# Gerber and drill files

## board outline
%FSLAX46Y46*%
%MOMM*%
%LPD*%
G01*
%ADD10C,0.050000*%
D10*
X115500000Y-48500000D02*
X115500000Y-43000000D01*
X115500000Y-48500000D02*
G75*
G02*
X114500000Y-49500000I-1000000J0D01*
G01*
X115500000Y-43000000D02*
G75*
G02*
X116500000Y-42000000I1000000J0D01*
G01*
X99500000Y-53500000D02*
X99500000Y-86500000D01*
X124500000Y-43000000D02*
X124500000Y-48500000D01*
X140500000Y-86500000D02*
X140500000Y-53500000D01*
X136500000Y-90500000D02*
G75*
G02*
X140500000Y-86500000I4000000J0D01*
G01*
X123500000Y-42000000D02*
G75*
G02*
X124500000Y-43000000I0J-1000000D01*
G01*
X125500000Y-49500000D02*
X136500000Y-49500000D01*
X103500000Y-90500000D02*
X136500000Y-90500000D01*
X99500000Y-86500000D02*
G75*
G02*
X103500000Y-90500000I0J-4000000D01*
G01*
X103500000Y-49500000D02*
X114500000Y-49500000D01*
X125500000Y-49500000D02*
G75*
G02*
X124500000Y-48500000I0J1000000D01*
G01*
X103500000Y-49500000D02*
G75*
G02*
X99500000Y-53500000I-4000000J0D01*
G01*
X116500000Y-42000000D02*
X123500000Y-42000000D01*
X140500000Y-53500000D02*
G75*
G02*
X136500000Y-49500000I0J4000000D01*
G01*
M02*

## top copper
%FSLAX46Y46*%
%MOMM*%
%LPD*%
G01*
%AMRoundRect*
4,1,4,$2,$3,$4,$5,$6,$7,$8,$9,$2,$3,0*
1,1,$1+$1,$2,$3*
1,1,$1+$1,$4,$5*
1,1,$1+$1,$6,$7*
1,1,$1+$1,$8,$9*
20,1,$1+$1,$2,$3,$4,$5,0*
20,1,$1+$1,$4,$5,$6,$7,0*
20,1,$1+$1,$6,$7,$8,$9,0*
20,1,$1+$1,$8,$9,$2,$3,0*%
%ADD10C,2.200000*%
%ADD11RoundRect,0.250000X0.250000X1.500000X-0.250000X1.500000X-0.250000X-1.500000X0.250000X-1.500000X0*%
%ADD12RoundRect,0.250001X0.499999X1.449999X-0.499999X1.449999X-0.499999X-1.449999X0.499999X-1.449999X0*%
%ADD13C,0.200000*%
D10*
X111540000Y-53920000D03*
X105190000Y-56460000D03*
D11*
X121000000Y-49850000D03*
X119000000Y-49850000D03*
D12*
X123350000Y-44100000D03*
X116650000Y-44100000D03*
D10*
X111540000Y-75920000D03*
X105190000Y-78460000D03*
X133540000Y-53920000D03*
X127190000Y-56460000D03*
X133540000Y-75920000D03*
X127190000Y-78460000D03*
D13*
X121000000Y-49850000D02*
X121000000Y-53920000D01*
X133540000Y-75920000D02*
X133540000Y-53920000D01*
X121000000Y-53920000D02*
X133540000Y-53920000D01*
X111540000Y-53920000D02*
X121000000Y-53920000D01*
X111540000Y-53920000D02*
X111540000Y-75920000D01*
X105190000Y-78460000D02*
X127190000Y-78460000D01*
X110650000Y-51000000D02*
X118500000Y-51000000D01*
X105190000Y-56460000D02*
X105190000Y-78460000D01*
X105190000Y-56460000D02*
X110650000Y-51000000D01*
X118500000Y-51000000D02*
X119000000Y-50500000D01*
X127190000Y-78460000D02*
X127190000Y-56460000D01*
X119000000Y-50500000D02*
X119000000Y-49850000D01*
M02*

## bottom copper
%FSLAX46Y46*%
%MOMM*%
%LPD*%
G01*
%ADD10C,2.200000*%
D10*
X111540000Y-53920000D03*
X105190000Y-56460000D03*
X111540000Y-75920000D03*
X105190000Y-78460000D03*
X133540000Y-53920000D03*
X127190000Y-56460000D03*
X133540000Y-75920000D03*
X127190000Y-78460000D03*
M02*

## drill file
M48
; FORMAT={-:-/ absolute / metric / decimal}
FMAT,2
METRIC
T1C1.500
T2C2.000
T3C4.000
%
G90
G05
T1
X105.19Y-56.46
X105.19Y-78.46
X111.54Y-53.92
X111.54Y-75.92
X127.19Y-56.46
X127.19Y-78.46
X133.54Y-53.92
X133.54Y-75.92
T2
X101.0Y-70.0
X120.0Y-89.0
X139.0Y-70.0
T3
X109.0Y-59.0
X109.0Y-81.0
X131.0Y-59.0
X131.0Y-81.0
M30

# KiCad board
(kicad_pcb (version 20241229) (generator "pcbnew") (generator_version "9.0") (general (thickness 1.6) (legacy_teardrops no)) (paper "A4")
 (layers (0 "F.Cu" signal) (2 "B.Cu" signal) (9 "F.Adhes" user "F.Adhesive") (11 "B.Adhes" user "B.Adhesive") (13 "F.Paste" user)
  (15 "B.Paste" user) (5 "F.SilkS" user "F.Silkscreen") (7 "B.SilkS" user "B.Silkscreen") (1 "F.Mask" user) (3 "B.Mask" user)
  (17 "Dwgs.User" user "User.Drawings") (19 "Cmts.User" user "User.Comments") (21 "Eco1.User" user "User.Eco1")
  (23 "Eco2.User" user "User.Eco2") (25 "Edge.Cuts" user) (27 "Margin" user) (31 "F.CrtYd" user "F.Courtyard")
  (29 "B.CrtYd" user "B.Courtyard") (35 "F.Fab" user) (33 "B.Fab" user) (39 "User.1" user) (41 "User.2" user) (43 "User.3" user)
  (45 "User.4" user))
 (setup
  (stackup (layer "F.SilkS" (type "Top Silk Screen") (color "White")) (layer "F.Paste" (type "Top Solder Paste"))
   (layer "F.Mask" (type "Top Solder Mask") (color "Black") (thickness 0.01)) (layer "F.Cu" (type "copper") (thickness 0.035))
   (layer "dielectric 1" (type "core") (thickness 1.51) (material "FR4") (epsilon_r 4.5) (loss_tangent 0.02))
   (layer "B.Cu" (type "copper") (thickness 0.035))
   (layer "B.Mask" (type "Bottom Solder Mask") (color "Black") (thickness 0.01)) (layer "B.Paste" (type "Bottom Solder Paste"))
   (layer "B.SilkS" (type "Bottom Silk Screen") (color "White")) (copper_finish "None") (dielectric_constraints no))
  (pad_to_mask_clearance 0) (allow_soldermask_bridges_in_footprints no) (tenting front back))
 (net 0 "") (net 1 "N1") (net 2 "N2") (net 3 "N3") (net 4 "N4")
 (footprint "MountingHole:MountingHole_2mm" (layer "F.Cu") (at 139 70)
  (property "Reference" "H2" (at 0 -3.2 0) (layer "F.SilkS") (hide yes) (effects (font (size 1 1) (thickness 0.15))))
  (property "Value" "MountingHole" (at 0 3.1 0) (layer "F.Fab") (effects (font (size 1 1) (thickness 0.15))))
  (pad "" np_thru_hole circle (at 0 0) (size 2 2) (drill 2) (layers "*.Cu" "*.Mask")))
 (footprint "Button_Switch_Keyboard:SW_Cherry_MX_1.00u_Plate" (layer "F.Cu") (at 111.54 53.92)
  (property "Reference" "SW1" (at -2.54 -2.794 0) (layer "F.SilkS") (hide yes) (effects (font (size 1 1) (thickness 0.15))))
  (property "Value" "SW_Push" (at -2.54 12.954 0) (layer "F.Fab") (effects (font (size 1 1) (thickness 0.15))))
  (pad "" np_thru_hole circle (at -2.54 5.08) (size 4 4) (drill 4) (layers "*.Cu" "*.Mask"))
  (pad "1" thru_hole circle (at 0 0) (size 2.2 2.2) (drill 1.5) (layers "*.Cu" "*.Mask") (remove_unused_layers no) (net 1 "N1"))
  (pad "2" thru_hole circle (at -6.35 2.54) (size 2.2 2.2) (drill 1.5) (layers "*.Cu" "*.Mask") (remove_unused_layers no) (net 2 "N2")))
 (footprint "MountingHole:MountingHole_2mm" (layer "F.Cu") (at 120 89)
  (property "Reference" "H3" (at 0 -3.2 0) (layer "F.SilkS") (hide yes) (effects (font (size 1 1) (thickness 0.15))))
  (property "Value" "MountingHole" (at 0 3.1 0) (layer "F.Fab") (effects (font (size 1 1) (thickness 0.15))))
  (pad "" np_thru_hole circle (at 0 0) (size 2 2) (drill 2) (layers "*.Cu" "*.Mask")))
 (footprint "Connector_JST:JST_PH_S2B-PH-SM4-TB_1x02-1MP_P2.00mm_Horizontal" (layer "F.Cu") (at 120 47 180)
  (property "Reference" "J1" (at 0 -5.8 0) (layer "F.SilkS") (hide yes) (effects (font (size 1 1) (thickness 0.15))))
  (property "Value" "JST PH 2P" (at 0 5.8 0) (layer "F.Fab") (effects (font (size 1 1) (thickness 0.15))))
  (pad "1" smd roundrect (at -1 -2.85 180) (size 1 3.5) (layers "F.Cu" "F.Mask" "F.Paste") (roundrect_rratio 0.25) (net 1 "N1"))
  (pad "2" smd roundrect (at 1 -2.85 180) (size 1 3.5) (layers "F.Cu" "F.Mask" "F.Paste") (roundrect_rratio 0.25) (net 2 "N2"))
  (pad "MP" smd roundrect (at -3.35 2.9 180) (size 1.5 3.4) (layers "F.Cu" "F.Mask" "F.Paste") (roundrect_rratio 0.166667) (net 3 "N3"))
  (pad "MP" smd roundrect (at 3.35 2.9 180) (size 1.5 3.4) (layers "F.Cu" "F.Mask" "F.Paste") (roundrect_rratio 0.166667) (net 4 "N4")))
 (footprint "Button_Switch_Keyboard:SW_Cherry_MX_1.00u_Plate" (layer "F.Cu") (at 111.54 75.92)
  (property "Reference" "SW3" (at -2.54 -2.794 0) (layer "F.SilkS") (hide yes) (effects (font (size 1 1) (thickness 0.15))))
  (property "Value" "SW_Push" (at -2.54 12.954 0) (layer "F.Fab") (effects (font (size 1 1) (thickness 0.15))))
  (pad "" np_thru_hole circle (at -2.54 5.08) (size 4 4) (drill 4) (layers "*.Cu" "*.Mask"))
  (pad "1" thru_hole circle (at 0 0) (size 2.2 2.2) (drill 1.5) (layers "*.Cu" "*.Mask") (remove_unused_layers no) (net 1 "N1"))
  (pad "2" thru_hole circle (at -6.35 2.54) (size 2.2 2.2) (drill 1.5) (layers "*.Cu" "*.Mask") (remove_unused_layers no) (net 2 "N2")))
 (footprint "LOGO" (layer "F.Cu") (at 126.5 70.1)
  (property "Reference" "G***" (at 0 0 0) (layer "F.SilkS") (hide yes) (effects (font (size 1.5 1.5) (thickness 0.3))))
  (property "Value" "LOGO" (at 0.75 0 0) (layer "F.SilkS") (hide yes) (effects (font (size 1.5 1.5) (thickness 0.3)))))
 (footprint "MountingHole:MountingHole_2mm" (layer "F.Cu") (at 101 70)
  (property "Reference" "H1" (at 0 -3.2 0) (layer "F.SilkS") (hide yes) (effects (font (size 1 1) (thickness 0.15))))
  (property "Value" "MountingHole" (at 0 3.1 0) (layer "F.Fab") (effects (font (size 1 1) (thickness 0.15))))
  (pad "" np_thru_hole circle (at 0 0) (size 2 2) (drill 2) (layers "*.Cu" "*.Mask")))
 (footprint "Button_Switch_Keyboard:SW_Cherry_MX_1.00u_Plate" (layer "F.Cu") (at 133.54 53.92)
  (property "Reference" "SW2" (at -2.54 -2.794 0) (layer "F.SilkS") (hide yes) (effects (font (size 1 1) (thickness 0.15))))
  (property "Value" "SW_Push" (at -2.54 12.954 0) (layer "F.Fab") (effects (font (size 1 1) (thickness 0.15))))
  (pad "" np_thru_hole circle (at -2.54 5.08) (size 4 4) (drill 4) (layers "*.Cu" "*.Mask"))
  (pad "1" thru_hole circle (at 0 0) (size 2.2 2.2) (drill 1.5) (layers "*.Cu" "*.Mask") (remove_unused_layers no) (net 1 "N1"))
  (pad "2" thru_hole circle (at -6.35 2.54) (size 2.2 2.2) (drill 1.5) (layers "*.Cu" "*.Mask") (remove_unused_layers no) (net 2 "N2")))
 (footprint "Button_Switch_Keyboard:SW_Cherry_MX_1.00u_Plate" (layer "F.Cu") (at 133.54 75.92)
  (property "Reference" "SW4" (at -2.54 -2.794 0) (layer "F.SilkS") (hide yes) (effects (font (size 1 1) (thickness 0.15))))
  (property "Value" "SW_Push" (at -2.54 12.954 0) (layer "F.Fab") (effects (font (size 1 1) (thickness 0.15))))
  (pad "" np_thru_hole circle (at -2.54 5.08) (size 4 4) (drill 4) (layers "*.Cu" "*.Mask"))
  (pad "1" thru_hole circle (at 0 0) (size 2.2 2.2) (drill 1.5) (layers "*.Cu" "*.Mask") (remove_unused_layers no) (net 1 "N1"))
  (pad "2" thru_hole circle (at -6.35 2.54) (size 2.2 2.2) (drill 1.5) (layers "*.Cu" "*.Mask") (remove_unused_layers no) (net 2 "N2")))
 (gr_line (start 115.5 48.5) (end 115.5 43) (stroke (width 0.05) (type default)) (layer "Edge.Cuts"))
 (gr_arc (start 115.5 48.5) (mid 115.207107 49.207107) (end 114.5 49.5) (stroke (width 0.05) (type default)) (layer "Edge.Cuts"))
 (gr_arc (start 115.5 43) (mid 115.792893 42.292893) (end 116.5 42) (stroke (width 0.05) (type default)) (layer "Edge.Cuts"))
 (gr_line (start 99.5 53.5) (end 99.5 86.5) (stroke (width 0.05) (type default)) (layer "Edge.Cuts"))
 (gr_line (start 124.5 43) (end 124.5 48.5) (stroke (width 0.05) (type default)) (layer "Edge.Cuts"))
 (gr_line (start 140.5 86.5) (end 140.5 53.5) (stroke (width 0.05) (type default)) (layer "Edge.Cuts"))
 (gr_arc (start 136.5 90.5) (mid 137.671573 87.671573) (end 140.5 86.5) (stroke (width 0.05) (type default)) (layer "Edge.Cuts"))
 (gr_arc (start 123.5 42) (mid 124.207107 42.292893) (end 124.5 43) (stroke (width 0.05) (type default)) (layer "Edge.Cuts"))
 (gr_line (start 125.5 49.5) (end 136.5 49.5) (stroke (width 0.05) (type default)) (layer "Edge.Cuts"))
 (gr_line (start 103.5 90.5) (end 136.5 90.5) (stroke (width 0.05) (type default)) (layer "Edge.Cuts"))
 (gr_arc (start 99.5 86.5) (mid 102.328427 87.671573) (end 103.5 90.5) (stroke (width 0.05) (type default)) (layer "Edge.Cuts"))
 (gr_line (start 103.5 49.5) (end 114.5 49.5) (stroke (width 0.05) (type default)) (layer "Edge.Cuts"))
 (gr_arc (start 125.5 49.5) (mid 124.792893 49.207107) (end 124.5 48.5) (stroke (width 0.05) (type default)) (layer "Edge.Cuts"))
 (gr_arc (start 103.5 49.5) (mid 102.328427 52.328427) (end 99.5 53.5) (stroke (width 0.05) (type default)) (layer "Edge.Cuts"))
 (gr_line (start 116.5 42) (end 123.5 42) (stroke (width 0.05) (type default)) (layer "Edge.Cuts"))
 (gr_arc (start 140.5 53.5) (mid 137.671573 52.328427) (end 136.5 49.5) (stroke (width 0.05) (type default)) (layer "Edge.Cuts"))
 (segment (start 121 49.85) (end 121 53.92) (width 0.2) (layer "F.Cu") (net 1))
 (segment (start 133.54 75.92) (end 133.54 53.92) (width 0.2) (layer "F.Cu") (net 1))
 (segment (start 121 53.92) (end 133.54 53.92) (width 0.2) (layer "F.Cu") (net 1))
 (segment (start 111.54 53.92) (end 121 53.92) (width 0.2) (layer "F.Cu") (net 1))
 (segment (start 111.54 53.92) (end 111.54 75.92) (width 0.2) (layer "F.Cu") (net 1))
 (segment (start 105.19 78.46) (end 127.19 78.46) (width 0.2) (layer "F.Cu") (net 2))
 (segment (start 110.65 51) (end 118.5 51) (width 0.2) (layer "F.Cu") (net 2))
 (segment (start 105.19 56.46) (end 105.19 78.46) (width 0.2) (layer "F.Cu") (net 2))
 (segment (start 105.19 56.46) (end 110.65 51) (width 0.2) (layer "F.Cu") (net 2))
 (segment (start 118.5 51) (end 119 50.5) (width 0.2) (layer "F.Cu") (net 2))
 (segment (start 127.19 78.46) (end 127.19 56.46) (width 0.2) (layer "F.Cu") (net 2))
 (segment (start 119 50.5) (end 119 49.85) (width 0.2) (layer "F.Cu") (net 2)))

